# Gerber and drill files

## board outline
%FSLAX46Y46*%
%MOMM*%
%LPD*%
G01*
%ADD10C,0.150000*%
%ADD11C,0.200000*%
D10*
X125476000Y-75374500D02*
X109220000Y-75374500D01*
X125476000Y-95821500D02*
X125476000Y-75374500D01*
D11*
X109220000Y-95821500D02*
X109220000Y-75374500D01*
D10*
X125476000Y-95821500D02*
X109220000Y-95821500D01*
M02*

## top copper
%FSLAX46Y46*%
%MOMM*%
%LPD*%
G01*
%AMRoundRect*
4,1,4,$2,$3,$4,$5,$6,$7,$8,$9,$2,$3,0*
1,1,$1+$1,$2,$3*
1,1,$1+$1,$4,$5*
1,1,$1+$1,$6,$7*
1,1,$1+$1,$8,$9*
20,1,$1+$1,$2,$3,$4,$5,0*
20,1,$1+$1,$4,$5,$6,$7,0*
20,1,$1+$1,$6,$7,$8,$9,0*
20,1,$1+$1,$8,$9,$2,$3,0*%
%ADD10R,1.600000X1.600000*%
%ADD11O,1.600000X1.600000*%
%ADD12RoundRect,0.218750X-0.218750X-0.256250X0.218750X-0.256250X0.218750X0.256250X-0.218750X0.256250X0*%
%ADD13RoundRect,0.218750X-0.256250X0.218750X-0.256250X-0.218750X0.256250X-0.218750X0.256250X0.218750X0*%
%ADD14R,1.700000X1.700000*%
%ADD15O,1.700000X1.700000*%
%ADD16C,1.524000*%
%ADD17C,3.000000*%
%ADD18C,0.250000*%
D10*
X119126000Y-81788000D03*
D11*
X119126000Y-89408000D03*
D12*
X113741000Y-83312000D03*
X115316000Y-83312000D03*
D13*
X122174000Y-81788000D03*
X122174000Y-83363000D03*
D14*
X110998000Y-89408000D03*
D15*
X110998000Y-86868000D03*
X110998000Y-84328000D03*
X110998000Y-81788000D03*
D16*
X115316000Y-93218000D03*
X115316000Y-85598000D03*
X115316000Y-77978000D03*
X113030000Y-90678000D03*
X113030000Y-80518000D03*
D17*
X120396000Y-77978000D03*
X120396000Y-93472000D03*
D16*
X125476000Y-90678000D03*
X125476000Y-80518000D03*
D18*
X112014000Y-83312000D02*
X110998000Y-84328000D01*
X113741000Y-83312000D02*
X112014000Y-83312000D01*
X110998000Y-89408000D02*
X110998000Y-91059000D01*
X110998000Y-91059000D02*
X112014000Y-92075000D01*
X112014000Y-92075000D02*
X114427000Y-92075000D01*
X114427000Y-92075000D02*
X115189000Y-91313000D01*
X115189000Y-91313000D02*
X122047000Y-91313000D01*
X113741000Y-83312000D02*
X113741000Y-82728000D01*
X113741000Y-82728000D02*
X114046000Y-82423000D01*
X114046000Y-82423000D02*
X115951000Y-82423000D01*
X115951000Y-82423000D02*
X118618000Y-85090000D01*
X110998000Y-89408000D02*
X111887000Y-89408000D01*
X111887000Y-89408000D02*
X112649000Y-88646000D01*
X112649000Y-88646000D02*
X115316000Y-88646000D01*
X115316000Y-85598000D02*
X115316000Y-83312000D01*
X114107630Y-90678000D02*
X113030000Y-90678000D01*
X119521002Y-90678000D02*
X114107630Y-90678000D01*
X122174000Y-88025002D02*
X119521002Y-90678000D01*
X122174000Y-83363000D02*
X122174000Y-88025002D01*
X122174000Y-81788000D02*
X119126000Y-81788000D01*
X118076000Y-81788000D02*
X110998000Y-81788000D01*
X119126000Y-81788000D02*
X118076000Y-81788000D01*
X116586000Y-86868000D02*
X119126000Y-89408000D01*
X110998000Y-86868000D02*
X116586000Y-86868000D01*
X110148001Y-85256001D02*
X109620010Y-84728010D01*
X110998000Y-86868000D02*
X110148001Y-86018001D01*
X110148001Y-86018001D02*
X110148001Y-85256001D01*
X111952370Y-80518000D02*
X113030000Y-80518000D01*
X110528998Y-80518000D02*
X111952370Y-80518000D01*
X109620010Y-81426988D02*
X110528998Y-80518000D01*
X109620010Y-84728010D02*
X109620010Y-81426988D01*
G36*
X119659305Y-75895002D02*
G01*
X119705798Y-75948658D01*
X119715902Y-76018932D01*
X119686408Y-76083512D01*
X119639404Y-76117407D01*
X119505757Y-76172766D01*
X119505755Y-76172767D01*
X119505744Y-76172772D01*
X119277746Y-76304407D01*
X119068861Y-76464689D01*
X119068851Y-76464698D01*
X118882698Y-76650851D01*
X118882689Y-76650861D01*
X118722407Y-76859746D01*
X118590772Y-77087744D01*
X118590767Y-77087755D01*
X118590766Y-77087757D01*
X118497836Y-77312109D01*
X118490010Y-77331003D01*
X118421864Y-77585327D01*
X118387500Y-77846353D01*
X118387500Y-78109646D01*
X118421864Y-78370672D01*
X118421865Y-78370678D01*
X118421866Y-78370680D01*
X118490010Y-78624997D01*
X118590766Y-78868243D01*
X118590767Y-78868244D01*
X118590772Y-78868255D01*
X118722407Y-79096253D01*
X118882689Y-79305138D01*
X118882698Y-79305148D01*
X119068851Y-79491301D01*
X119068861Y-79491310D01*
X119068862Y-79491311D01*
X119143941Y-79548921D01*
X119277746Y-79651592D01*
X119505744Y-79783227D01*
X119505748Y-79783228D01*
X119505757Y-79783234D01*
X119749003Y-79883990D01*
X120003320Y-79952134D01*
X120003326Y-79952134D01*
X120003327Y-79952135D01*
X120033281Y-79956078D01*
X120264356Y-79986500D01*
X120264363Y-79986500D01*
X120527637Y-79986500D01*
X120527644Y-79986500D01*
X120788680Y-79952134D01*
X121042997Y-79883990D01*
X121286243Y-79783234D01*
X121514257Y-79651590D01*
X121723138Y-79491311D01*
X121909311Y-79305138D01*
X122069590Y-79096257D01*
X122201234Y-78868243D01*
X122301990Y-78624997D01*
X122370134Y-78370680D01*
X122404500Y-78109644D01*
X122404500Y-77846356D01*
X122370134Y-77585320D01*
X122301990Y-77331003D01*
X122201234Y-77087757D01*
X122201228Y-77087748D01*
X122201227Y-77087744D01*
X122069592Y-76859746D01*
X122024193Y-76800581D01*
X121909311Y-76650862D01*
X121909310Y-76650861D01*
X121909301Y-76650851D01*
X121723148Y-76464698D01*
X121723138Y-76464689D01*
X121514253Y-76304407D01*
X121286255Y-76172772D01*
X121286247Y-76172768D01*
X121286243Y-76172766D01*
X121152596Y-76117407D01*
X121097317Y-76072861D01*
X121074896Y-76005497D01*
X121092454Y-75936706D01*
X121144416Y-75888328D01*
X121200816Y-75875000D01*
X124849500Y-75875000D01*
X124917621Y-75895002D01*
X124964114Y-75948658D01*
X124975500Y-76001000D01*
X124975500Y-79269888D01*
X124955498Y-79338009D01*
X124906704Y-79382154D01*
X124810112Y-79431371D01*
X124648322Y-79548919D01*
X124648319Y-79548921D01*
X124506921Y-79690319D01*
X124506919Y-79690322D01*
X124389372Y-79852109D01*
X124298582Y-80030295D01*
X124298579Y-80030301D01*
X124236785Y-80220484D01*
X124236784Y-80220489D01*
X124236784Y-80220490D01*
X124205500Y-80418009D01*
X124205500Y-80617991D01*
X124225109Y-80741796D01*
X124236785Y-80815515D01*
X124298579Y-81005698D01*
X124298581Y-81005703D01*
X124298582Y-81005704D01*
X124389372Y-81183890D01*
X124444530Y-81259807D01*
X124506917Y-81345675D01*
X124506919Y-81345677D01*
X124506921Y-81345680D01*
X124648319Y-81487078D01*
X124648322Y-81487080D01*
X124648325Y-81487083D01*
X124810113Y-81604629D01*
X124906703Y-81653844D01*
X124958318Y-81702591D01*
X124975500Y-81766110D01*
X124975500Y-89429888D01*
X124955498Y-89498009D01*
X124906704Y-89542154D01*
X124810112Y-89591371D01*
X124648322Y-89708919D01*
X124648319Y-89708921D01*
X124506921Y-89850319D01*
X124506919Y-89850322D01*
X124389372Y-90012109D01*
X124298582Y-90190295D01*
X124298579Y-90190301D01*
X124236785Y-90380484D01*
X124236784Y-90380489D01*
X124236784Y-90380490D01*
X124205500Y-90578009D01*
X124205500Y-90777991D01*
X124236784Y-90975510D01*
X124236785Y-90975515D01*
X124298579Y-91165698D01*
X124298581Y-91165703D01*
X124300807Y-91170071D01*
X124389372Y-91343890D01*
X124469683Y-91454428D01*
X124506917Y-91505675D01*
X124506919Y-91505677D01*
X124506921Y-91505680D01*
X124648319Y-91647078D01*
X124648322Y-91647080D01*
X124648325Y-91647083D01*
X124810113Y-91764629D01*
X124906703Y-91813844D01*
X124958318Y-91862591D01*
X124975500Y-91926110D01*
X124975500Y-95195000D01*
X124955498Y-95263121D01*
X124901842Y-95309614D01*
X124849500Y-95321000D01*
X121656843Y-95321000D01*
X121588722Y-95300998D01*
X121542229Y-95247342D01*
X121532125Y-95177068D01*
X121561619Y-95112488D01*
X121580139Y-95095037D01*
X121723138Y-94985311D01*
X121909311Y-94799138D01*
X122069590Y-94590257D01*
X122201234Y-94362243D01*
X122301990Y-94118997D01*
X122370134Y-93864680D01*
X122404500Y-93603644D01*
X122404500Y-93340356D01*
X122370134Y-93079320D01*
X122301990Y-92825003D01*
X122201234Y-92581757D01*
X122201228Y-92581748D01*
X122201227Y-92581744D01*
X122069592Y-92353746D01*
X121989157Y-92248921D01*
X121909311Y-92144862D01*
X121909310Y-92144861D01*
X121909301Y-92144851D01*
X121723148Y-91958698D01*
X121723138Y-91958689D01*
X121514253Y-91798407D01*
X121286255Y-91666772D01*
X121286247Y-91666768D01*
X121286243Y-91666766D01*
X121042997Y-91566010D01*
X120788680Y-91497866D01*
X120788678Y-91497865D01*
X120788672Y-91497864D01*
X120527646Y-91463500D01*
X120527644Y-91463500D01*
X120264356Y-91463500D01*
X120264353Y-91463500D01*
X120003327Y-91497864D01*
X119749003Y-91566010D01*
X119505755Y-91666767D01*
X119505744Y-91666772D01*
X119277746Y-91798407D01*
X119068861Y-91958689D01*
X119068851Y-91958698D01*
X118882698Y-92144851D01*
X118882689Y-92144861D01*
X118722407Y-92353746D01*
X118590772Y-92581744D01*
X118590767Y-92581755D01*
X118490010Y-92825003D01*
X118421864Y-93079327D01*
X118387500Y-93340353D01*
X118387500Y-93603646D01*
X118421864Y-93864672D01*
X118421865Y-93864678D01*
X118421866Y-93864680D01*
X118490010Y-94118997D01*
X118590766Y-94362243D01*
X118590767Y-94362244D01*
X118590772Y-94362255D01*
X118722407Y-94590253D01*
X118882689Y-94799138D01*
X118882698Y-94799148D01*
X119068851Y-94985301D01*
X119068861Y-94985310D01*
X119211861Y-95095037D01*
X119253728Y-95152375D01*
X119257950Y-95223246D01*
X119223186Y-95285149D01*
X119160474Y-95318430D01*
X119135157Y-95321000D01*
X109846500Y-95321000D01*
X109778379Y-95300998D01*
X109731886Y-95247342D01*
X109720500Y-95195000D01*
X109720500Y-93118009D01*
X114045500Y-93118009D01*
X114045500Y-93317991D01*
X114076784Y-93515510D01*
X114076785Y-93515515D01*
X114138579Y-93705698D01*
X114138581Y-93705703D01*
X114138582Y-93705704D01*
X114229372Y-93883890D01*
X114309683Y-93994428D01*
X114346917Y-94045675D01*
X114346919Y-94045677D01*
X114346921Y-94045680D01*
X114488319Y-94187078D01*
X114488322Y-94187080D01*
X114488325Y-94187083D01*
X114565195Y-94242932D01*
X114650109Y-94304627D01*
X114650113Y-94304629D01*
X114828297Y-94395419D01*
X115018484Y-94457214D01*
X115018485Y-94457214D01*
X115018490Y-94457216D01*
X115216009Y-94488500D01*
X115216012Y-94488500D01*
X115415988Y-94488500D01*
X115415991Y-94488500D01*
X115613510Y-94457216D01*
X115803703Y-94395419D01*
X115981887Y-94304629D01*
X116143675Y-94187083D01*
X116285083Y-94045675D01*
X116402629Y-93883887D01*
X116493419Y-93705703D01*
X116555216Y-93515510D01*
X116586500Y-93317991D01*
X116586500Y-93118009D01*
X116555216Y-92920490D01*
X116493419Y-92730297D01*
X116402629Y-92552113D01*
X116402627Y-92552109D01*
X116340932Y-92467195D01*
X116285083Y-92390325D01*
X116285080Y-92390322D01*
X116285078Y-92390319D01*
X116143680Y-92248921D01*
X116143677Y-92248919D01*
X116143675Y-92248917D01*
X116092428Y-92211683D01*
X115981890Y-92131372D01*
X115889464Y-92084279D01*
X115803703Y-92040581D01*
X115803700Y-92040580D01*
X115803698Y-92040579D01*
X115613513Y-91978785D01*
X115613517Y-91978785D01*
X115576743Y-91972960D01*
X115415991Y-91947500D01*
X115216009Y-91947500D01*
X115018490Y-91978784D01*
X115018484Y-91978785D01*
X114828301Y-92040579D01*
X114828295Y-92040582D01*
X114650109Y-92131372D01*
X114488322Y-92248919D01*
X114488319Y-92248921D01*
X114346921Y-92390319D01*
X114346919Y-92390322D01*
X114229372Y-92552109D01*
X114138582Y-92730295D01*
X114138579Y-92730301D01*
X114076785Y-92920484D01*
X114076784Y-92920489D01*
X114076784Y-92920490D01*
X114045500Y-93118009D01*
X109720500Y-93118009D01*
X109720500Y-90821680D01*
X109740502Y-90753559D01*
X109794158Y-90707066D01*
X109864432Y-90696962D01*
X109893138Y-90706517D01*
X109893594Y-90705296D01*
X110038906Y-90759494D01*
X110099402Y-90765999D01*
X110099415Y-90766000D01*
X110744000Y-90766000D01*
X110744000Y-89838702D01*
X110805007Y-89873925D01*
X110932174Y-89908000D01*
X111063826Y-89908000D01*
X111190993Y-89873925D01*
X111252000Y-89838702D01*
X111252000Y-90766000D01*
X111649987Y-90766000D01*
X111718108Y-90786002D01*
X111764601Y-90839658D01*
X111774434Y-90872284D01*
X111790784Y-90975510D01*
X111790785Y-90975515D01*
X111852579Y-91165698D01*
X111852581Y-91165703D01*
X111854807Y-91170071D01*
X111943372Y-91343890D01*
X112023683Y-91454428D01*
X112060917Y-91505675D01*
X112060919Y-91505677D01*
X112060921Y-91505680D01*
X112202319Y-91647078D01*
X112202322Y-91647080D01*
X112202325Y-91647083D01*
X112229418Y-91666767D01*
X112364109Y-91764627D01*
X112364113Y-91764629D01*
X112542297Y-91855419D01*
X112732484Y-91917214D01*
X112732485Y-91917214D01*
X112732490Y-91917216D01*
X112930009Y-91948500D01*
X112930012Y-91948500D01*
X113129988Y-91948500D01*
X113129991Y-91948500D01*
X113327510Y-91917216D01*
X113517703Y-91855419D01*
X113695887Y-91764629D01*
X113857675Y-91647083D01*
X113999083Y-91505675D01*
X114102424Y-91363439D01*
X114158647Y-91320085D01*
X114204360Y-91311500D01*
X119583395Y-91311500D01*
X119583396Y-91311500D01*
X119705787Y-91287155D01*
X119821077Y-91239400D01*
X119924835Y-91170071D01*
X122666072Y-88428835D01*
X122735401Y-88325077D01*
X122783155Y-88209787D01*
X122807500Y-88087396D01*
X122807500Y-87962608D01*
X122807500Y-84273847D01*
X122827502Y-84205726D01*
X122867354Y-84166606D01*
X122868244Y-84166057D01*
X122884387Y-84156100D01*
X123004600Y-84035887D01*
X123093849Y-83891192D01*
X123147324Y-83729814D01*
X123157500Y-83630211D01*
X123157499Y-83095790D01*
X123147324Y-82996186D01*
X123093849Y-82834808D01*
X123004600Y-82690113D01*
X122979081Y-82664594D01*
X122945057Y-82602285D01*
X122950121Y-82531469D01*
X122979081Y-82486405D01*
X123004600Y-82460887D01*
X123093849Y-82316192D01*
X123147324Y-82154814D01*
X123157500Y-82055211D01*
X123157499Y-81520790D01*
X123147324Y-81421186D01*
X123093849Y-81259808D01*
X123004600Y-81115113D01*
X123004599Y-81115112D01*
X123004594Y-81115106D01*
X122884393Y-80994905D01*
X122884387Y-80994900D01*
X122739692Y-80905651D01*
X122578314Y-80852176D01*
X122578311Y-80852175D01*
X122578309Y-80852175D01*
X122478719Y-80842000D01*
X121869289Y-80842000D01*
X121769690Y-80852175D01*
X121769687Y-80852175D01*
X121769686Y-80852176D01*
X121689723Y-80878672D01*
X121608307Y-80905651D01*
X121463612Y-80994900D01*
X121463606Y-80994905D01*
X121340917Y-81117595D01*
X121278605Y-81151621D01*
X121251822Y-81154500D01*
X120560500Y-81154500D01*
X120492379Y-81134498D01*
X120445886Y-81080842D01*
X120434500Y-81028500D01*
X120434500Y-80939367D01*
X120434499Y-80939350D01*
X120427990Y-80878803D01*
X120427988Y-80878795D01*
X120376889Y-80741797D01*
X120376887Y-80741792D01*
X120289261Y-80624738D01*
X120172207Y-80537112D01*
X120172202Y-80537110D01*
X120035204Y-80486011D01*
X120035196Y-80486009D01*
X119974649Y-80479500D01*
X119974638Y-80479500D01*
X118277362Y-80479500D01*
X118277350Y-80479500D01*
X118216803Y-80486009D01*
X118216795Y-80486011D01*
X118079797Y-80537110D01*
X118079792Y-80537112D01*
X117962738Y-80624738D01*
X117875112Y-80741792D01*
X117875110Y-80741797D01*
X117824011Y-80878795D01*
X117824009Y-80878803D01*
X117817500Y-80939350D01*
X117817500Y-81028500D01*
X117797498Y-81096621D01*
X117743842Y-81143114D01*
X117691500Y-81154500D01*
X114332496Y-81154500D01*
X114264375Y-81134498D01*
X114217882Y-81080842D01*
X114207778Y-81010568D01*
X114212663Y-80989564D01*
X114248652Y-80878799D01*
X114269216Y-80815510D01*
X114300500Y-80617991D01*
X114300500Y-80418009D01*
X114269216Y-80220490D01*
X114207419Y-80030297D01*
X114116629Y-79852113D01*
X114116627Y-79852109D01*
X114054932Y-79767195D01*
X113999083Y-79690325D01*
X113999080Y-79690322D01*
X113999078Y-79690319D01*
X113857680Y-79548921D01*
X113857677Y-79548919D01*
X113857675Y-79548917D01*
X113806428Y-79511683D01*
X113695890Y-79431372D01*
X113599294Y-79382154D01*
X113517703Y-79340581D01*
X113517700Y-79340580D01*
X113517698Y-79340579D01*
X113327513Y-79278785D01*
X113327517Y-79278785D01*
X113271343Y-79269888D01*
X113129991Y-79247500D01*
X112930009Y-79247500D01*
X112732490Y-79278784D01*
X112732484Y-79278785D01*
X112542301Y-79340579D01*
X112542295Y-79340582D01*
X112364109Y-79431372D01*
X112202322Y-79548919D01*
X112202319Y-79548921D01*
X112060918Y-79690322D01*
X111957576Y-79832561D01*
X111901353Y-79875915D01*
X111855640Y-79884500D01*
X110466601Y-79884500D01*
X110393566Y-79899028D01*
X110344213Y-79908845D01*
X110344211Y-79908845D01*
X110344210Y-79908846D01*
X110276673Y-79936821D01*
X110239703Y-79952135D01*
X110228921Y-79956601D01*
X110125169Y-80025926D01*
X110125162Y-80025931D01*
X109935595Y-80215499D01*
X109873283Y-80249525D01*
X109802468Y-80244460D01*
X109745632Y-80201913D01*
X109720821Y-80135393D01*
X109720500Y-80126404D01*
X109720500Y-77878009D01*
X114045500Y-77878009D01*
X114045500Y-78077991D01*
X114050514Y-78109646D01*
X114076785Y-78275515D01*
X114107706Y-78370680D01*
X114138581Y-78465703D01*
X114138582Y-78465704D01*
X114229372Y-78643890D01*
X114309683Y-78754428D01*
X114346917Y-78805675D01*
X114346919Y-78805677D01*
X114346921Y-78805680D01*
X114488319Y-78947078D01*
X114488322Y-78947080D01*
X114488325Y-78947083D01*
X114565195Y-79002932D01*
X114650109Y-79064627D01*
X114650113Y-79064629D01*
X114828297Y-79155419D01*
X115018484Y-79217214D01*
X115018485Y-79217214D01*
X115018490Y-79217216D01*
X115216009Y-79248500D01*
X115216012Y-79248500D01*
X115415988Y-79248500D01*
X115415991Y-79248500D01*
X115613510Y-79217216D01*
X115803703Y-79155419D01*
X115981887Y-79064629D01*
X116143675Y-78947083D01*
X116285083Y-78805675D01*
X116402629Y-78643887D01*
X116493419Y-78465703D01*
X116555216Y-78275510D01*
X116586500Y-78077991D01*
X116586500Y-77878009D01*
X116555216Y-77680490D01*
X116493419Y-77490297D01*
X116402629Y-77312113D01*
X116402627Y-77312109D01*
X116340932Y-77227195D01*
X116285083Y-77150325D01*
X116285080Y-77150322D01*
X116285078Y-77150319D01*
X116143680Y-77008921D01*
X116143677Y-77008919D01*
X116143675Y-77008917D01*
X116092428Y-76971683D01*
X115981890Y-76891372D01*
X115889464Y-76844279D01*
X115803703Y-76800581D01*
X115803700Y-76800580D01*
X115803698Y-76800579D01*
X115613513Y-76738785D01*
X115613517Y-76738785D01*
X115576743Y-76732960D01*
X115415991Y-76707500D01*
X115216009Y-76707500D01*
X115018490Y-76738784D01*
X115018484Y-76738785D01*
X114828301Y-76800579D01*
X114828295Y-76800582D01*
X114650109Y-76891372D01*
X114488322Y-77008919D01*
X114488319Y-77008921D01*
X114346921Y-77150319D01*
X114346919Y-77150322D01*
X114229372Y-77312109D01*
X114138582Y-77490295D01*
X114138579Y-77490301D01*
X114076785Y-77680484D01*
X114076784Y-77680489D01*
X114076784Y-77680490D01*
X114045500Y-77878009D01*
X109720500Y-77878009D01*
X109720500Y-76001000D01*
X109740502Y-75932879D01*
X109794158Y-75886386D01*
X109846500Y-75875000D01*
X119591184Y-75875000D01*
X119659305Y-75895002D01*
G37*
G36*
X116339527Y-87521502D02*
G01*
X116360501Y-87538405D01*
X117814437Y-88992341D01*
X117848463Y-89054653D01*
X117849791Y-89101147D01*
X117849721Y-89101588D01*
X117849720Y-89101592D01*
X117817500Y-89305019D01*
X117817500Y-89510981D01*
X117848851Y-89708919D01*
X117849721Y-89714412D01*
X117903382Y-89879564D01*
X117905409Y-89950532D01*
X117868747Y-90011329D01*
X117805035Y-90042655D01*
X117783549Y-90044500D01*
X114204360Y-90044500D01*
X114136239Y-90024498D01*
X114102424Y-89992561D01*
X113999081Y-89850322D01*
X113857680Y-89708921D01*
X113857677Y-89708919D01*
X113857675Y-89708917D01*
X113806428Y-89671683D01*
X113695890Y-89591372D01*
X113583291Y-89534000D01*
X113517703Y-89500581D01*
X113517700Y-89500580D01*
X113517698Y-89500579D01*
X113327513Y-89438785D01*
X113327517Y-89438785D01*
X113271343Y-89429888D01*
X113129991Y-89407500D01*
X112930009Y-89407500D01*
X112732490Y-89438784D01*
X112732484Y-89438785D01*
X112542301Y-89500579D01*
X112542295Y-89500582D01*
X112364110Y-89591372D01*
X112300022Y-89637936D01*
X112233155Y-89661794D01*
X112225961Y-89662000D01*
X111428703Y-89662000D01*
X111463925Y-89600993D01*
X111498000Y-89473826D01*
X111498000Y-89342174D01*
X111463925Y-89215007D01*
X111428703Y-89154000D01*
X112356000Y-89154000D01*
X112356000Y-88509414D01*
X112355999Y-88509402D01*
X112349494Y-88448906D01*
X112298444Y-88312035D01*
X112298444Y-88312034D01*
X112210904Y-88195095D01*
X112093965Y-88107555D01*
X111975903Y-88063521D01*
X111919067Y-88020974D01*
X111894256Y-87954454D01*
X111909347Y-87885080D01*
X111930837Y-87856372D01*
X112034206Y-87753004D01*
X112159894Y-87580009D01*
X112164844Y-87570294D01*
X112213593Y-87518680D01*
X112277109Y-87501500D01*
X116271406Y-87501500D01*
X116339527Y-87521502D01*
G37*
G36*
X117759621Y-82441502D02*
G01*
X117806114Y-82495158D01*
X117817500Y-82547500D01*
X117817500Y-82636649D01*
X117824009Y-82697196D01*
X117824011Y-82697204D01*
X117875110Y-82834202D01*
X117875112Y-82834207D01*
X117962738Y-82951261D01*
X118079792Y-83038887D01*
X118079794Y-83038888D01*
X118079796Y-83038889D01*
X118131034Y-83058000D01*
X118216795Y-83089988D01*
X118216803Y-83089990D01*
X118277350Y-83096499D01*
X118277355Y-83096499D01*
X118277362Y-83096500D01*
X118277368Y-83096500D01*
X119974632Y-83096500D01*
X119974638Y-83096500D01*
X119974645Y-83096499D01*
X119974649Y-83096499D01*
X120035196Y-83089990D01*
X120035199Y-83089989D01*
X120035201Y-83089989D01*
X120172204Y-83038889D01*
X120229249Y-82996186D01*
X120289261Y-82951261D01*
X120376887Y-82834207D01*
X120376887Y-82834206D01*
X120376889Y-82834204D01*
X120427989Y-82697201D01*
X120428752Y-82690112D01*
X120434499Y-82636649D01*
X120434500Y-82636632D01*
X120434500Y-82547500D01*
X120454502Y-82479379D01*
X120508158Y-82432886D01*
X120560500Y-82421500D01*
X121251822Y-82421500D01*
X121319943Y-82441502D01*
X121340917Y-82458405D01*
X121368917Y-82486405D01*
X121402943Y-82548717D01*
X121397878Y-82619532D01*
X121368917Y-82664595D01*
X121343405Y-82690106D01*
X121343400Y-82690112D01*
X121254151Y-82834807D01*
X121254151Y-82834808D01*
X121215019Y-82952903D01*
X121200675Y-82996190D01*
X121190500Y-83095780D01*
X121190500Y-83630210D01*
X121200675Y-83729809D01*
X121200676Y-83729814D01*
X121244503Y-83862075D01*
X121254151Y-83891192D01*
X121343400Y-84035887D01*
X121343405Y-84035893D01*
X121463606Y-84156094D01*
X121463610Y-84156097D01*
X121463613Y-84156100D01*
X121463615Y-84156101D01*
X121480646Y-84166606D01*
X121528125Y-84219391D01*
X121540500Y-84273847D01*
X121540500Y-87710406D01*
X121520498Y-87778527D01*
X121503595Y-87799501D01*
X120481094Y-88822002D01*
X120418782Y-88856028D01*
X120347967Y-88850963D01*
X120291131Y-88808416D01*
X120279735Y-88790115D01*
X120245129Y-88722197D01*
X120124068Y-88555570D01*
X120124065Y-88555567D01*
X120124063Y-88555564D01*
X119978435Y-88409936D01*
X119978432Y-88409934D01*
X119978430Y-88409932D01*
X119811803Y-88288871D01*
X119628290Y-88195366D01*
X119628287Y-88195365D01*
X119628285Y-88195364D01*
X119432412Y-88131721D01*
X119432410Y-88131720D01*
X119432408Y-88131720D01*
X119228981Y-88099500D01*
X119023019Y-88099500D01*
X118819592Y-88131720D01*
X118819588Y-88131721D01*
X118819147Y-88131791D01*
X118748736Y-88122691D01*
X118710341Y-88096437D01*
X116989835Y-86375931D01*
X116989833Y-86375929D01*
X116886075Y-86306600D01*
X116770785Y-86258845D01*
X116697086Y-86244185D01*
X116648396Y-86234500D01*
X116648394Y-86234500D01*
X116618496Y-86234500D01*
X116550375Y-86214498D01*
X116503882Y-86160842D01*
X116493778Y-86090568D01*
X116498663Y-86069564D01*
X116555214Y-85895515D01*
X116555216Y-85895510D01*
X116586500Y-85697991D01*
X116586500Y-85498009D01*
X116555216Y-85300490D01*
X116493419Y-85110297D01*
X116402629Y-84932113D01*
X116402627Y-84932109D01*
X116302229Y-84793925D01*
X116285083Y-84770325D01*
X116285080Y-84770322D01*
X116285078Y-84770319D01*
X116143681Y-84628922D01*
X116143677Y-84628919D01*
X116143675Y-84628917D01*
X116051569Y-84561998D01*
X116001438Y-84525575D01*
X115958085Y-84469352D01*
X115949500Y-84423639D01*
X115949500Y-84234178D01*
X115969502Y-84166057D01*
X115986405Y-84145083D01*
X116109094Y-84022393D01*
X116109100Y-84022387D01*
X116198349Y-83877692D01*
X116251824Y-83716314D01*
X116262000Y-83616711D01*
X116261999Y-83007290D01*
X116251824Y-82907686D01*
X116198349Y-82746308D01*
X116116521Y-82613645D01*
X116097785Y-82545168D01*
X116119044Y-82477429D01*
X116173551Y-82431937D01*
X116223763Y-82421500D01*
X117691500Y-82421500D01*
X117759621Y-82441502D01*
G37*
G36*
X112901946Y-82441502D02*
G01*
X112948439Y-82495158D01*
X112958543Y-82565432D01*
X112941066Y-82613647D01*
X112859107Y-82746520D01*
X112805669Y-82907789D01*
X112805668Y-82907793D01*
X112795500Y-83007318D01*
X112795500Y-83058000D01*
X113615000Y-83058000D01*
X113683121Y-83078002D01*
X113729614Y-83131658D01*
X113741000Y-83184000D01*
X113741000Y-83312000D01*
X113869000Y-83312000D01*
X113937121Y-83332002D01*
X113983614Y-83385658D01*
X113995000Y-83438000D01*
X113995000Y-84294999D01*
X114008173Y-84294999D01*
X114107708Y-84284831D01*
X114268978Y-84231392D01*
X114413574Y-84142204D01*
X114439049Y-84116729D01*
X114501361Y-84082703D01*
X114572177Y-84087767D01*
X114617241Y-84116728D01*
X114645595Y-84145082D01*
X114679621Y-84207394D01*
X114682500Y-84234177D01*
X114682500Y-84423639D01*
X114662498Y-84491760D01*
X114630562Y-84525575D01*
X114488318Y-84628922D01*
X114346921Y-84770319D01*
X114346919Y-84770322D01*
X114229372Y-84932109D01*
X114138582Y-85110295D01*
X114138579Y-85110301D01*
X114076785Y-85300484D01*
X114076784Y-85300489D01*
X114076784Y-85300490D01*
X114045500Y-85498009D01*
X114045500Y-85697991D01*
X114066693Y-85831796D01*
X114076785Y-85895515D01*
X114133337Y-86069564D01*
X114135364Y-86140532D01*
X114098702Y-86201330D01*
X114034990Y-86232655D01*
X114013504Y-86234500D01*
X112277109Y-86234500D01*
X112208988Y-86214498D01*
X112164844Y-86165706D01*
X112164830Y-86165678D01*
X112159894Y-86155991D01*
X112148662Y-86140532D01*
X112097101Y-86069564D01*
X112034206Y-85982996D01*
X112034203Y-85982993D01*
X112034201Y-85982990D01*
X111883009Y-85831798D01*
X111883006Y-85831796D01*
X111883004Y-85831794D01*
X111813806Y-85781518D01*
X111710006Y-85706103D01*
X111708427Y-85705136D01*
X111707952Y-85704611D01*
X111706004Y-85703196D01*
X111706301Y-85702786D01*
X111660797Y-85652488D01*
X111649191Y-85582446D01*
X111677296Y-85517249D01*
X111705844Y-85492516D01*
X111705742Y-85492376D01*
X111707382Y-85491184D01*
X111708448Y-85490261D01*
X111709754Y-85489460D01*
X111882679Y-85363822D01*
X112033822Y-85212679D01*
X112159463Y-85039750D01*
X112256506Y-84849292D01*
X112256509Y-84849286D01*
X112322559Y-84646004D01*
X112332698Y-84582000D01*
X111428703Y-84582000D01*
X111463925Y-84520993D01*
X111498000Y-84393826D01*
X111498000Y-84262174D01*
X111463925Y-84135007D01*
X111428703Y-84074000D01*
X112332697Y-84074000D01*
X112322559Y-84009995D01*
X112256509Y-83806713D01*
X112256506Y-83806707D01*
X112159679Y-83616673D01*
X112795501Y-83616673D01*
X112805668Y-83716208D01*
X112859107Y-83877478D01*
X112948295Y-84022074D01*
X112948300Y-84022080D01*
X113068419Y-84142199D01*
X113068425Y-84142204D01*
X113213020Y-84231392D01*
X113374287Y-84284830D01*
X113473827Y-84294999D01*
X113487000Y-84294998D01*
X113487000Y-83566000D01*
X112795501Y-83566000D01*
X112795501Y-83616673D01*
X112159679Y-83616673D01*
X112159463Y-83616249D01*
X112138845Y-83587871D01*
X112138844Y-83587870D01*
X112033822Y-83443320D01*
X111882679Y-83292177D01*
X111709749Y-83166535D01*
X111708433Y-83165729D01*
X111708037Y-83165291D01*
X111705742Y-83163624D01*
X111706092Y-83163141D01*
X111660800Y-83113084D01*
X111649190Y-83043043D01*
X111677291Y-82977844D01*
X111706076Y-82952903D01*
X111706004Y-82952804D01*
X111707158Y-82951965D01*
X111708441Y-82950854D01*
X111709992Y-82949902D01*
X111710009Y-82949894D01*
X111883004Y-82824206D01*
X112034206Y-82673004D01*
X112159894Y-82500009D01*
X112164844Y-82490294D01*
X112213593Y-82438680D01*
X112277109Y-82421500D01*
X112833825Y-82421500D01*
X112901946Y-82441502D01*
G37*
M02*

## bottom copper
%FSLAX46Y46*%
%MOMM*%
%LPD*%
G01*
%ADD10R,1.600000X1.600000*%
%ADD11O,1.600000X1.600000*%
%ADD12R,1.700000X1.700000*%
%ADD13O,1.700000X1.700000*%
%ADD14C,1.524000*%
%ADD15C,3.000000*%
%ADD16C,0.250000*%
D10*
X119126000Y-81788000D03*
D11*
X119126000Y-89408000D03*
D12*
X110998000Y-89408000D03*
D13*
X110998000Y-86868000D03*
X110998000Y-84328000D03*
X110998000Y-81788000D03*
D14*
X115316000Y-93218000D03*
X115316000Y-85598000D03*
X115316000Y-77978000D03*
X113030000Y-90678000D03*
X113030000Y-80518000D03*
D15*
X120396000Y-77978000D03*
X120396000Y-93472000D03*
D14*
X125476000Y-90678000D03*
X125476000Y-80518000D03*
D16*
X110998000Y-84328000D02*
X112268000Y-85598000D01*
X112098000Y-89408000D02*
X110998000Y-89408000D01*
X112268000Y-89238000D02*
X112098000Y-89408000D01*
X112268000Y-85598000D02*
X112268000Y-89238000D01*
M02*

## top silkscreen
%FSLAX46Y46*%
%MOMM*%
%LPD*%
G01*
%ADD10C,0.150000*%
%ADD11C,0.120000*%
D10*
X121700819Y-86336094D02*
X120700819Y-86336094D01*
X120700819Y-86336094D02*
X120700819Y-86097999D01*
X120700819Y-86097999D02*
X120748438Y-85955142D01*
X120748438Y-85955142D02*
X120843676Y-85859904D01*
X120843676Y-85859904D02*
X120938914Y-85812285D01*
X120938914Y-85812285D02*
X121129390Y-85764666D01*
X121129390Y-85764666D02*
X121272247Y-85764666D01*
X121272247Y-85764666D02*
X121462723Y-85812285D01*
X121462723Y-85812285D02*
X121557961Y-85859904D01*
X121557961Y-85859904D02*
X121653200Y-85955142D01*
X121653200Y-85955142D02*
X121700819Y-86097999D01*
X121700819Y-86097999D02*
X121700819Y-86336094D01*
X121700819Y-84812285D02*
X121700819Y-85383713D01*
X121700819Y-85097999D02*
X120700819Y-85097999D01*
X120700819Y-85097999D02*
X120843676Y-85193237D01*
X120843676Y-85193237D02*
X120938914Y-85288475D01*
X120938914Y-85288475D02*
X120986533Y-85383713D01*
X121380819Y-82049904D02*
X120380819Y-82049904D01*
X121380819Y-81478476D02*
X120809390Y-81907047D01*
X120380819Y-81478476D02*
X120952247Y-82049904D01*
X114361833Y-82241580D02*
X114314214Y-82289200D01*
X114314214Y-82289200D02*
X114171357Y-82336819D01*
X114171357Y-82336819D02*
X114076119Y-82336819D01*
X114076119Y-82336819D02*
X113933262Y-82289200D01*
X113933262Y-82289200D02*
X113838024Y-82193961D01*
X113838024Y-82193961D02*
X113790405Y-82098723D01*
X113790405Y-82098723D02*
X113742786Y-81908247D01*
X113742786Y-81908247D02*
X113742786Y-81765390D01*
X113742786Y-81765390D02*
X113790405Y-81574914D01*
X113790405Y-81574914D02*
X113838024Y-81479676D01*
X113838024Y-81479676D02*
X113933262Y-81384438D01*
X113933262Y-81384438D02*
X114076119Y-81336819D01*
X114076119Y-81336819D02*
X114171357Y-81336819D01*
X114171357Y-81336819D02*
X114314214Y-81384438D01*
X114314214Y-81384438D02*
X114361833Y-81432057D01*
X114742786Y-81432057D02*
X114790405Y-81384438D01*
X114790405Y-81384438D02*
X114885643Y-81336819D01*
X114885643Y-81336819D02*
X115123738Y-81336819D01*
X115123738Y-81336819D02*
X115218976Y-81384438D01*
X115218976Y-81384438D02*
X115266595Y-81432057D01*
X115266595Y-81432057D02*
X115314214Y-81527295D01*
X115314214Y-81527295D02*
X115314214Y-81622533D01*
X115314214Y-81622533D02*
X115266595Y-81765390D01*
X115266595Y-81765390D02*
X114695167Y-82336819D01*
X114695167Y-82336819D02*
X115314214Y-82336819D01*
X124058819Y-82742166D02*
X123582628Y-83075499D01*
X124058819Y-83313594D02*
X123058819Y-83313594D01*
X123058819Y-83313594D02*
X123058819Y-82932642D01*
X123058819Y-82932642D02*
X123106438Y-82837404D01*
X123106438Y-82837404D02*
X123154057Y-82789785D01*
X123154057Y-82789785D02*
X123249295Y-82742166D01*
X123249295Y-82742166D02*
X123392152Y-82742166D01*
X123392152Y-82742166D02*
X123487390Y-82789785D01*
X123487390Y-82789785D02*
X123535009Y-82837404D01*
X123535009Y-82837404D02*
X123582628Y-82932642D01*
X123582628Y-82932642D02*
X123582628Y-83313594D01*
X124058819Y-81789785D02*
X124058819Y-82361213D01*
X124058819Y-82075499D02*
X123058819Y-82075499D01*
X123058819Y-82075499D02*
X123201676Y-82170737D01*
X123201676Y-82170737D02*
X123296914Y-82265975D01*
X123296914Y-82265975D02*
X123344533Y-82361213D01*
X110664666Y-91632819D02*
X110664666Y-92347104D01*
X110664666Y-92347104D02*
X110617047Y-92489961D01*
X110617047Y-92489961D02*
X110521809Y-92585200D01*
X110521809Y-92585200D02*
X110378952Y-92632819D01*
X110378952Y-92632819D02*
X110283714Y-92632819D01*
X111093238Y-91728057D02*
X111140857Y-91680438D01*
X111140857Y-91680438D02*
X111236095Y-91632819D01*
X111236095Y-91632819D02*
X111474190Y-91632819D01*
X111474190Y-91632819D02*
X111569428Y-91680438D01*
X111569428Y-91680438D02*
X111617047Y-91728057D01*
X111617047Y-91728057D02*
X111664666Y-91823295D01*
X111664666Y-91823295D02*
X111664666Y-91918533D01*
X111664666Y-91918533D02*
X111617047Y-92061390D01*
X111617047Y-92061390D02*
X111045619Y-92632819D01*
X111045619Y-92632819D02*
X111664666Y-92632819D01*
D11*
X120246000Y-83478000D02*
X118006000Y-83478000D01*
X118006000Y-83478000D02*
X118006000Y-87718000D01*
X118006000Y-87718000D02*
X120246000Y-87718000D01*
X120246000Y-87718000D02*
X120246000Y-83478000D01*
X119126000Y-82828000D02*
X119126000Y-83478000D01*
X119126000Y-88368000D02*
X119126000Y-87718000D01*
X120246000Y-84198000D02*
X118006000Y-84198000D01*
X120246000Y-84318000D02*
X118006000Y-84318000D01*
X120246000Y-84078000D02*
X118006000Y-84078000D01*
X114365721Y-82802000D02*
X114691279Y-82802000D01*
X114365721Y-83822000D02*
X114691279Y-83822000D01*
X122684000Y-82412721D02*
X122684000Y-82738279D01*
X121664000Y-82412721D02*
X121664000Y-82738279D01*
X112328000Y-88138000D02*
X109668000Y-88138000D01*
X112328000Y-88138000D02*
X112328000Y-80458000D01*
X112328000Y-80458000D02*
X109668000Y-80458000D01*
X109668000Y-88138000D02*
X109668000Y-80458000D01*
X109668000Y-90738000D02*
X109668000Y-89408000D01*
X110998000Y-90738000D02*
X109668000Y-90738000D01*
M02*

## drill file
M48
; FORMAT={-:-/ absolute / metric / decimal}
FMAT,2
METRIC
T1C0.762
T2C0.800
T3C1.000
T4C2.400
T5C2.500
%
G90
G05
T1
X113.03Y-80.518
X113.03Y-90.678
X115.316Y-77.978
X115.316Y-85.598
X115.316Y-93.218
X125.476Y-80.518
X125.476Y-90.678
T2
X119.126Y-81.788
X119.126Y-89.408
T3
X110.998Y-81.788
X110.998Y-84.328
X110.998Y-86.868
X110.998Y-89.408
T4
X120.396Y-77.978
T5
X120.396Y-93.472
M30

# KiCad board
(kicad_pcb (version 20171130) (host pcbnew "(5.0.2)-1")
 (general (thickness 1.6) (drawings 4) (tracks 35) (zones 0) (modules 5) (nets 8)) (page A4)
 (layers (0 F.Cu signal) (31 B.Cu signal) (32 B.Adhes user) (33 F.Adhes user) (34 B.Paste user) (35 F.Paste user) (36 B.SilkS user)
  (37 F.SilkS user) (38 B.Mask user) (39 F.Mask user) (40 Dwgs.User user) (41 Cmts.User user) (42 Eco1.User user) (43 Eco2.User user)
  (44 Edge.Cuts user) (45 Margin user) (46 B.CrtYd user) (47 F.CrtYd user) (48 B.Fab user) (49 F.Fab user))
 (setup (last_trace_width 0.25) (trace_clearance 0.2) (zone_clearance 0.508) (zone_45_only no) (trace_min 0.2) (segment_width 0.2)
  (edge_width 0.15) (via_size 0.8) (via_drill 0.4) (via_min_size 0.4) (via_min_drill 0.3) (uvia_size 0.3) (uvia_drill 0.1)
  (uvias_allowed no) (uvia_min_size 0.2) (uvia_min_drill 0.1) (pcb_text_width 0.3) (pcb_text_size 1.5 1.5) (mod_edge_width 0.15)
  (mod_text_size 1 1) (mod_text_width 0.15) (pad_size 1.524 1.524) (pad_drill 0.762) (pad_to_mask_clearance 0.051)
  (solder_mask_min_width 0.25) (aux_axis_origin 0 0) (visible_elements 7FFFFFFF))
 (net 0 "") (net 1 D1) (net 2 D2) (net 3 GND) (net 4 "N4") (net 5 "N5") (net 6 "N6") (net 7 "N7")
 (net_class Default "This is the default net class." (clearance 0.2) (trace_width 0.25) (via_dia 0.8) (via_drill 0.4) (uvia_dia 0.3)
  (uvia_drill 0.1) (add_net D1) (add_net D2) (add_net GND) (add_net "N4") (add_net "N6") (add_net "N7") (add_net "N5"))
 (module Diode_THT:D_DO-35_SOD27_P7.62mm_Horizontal (layer F.Cu) (at 119.126 81.788 270)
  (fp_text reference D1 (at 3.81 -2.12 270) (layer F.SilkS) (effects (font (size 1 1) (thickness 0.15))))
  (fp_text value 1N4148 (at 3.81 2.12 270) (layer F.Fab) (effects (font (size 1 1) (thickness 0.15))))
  (fp_line (start 1.69 -1.12) (end 1.69 1.12) (layer F.SilkS) (width 0.12))
  (fp_line (start 1.69 1.12) (end 5.93 1.12) (layer F.SilkS) (width 0.12))
  (fp_line (start 5.93 1.12) (end 5.93 -1.12) (layer F.SilkS) (width 0.12))
  (fp_line (start 5.93 -1.12) (end 1.69 -1.12) (layer F.SilkS) (width 0.12))
  (fp_line (start 1.04 0) (end 1.69 0) (layer F.SilkS) (width 0.12))
  (fp_line (start 6.58 0) (end 5.93 0) (layer F.SilkS) (width 0.12))
  (fp_line (start 2.41 -1.12) (end 2.41 1.12) (layer F.SilkS) (width 0.12))
  (fp_line (start 2.53 -1.12) (end 2.53 1.12) (layer F.SilkS) (width 0.12))
  (fp_line (start 2.29 -1.12) (end 2.29 1.12) (layer F.SilkS) (width 0.12))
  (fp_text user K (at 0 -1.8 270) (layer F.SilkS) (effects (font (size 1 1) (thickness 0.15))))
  (pad 1 thru_hole rect (at 0 0 270) (size 1.6 1.6) (drill 0.8) (layers *.Cu *.Mask) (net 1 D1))
  (pad 2 thru_hole oval (at 7.62 0 270) (size 1.6 1.6) (drill 0.8) (layers *.Cu *.Mask) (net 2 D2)))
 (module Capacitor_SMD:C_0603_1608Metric (layer F.Cu) (at 114.5285 83.312)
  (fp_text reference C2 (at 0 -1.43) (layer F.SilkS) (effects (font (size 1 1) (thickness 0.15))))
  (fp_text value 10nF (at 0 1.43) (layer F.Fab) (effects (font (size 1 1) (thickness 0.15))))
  (fp_line (start -0.162779 -0.51) (end 0.162779 -0.51) (layer F.SilkS) (width 0.12))
  (fp_line (start -0.162779 0.51) (end 0.162779 0.51) (layer F.SilkS) (width 0.12))
  (pad 1 smd roundrect (at -0.7875 0) (size 0.875 0.95) (layers F.Cu F.Paste F.Mask) (roundrect_rratio 0.25) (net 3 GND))
  (pad 2 smd roundrect (at 0.7875 0) (size 0.875 0.95) (layers F.Cu F.Paste F.Mask) (roundrect_rratio 0.25) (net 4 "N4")))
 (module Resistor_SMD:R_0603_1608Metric (layer F.Cu) (at 122.174 82.5755 270)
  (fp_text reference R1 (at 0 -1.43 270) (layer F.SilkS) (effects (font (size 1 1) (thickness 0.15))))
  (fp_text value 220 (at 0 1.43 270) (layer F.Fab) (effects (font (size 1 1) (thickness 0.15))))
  (fp_line (start -0.162779 -0.51) (end 0.162779 -0.51) (layer F.SilkS) (width 0.12))
  (fp_line (start -0.162779 0.51) (end 0.162779 0.51) (layer F.SilkS) (width 0.12))
  (pad 1 smd roundrect (at -0.7875 0 270) (size 0.875 0.95) (layers F.Cu F.Paste F.Mask) (roundrect_rratio 0.25) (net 1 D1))
  (pad 2 smd roundrect (at 0.7875 0 270) (size 0.875 0.95) (layers F.Cu F.Paste F.Mask) (roundrect_rratio 0.25) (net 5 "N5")))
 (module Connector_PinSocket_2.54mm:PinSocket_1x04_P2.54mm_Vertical (layer F.Cu) (at 110.998 89.408 180)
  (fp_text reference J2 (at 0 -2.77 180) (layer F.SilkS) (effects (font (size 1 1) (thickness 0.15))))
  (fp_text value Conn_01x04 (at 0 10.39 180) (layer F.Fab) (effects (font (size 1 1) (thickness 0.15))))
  (fp_line (start -1.33 1.27) (end 1.33 1.27) (layer F.SilkS) (width 0.12))
  (fp_line (start -1.33 1.27) (end -1.33 8.95) (layer F.SilkS) (width 0.12))
  (fp_line (start -1.33 8.95) (end 1.33 8.95) (layer F.SilkS) (width 0.12))
  (fp_line (start 1.33 1.27) (end 1.33 8.95) (layer F.SilkS) (width 0.12))
  (fp_line (start 1.33 -1.33) (end 1.33 0) (layer F.SilkS) (width 0.12))
  (fp_line (start 0 -1.33) (end 1.33 -1.33) (layer F.SilkS) (width 0.12))
  (pad 1 thru_hole rect (at 0 0 180) (size 1.7 1.7) (drill 1) (layers *.Cu *.Mask) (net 3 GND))
  (pad 2 thru_hole oval (at 0 2.54 180) (size 1.7 1.7) (drill 1) (layers *.Cu *.Mask) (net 2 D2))
  (pad 3 thru_hole oval (at 0 5.08 180) (size 1.7 1.7) (drill 1) (layers *.Cu *.Mask) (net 3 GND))
  (pad 4 thru_hole oval (at 0 7.62 180) (size 1.7 1.7) (drill 1) (layers *.Cu *.Mask) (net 1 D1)))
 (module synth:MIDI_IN (layer B.Cu) (at 115.316 85.598 270)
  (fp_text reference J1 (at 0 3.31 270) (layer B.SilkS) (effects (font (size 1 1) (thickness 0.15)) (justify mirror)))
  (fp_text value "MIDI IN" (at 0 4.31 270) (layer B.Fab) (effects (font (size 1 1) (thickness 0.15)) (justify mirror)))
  (pad 1 thru_hole circle (at 7.62 0 270) (size 1.524 1.524) (drill 0.762) (layers *.Cu *.Mask) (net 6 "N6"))
  (pad 2 thru_hole circle (at 0 0 270) (size 1.524 1.524) (drill 0.762) (layers *.Cu *.Mask) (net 4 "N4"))
  (pad 3 thru_hole circle (at -7.62 0 270) (size 1.524 1.524) (drill 0.762) (layers *.Cu *.Mask) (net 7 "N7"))
  (pad 4 thru_hole circle (at 5.08 2.286 270) (size 1.524 1.524) (drill 0.762) (layers *.Cu *.Mask) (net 5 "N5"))
  (pad 5 thru_hole circle (at -5.08 2.286 270) (size 1.524 1.524) (drill 0.762) (layers *.Cu *.Mask) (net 2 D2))
  (pad "" thru_hole circle (at -7.62 -5.08 270) (size 3 3) (drill 2.4) (layers *.Cu *.Mask))
  (pad "" thru_hole circle (at 7.874 -5.08 270) (size 3 3) (drill 2.5) (layers *.Cu *.Mask))
  (pad "" thru_hole circle (at 5.08 -10.16 270) (size 1.524 1.524) (drill 0.762) (layers *.Cu *.Mask))
  (pad "" thru_hole circle (at -5.08 -10.16 270) (size 1.524 1.524) (drill 0.762) (layers *.Cu *.Mask)))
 (gr_line (start 125.476 75.3745) (end 109.22 75.3745) (layer Edge.Cuts) (width 0.15))
 (gr_line (start 125.476 95.8215) (end 125.476 75.3745) (layer Edge.Cuts) (width 0.15))
 (gr_line (start 109.22 95.8215) (end 109.22 75.3745) (layer Edge.Cuts) (width 0.2))
 (gr_line (start 125.476 95.8215) (end 109.22 95.8215) (layer Edge.Cuts) (width 0.15))
 (segment (start 112.014 83.312) (end 110.998 84.328) (width 0.25) (layer F.Cu) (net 3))
 (segment (start 113.741 83.312) (end 112.014 83.312) (width 0.25) (layer F.Cu) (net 3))
 (segment (start 110.998 84.328) (end 112.268 85.598) (width 0.25) (layer B.Cu) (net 3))
 (segment (start 112.098 89.408) (end 110.998 89.408) (width 0.25) (layer B.Cu) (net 3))
 (segment (start 112.268 89.238) (end 112.098 89.408) (width 0.25) (layer B.Cu) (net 3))
 (segment (start 112.268 85.598) (end 112.268 89.238) (width 0.25) (layer B.Cu) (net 3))
 (segment (start 110.998 89.408) (end 110.998 91.059) (width 0.25) (layer F.Cu) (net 3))
 (segment (start 110.998 91.059) (end 112.014 92.075) (width 0.25) (layer F.Cu) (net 3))
 (segment (start 112.014 92.075) (end 114.427 92.075) (width 0.25) (layer F.Cu) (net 3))
 (segment (start 114.427 92.075) (end 115.189 91.313) (width 0.25) (layer F.Cu) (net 3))
 (segment (start 115.189 91.313) (end 122.047 91.313) (width 0.25) (layer F.Cu) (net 3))
 (segment (start 113.741 83.312) (end 113.741 82.728) (width 0.25) (layer F.Cu) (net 3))
 (segment (start 113.741 82.728) (end 114.046 82.423) (width 0.25) (layer F.Cu) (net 3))
 (segment (start 114.046 82.423) (end 115.951 82.423) (width 0.25) (layer F.Cu) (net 3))
 (segment (start 115.951 82.423) (end 118.618 85.09) (width 0.25) (layer F.Cu) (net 3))
 (segment (start 110.998 89.408) (end 111.887 89.408) (width 0.25) (layer F.Cu) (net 3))
 (segment (start 111.887 89.408) (end 112.649 88.646) (width 0.25) (layer F.Cu) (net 3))
 (segment (start 112.649 88.646) (end 115.316 88.646) (width 0.25) (layer F.Cu) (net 3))
 (segment (start 115.316 85.598) (end 115.316 83.312) (width 0.25) (layer F.Cu) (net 4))
 (segment (start 114.10763 90.678) (end 113.03 90.678) (width 0.25) (layer F.Cu) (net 5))
 (segment (start 119.521002 90.678) (end 114.10763 90.678) (width 0.25) (layer F.Cu) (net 5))
 (segment (start 122.174 88.025002) (end 119.521002 90.678) (width 0.25) (layer F.Cu) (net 5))
 (segment (start 122.174 83.363) (end 122.174 88.025002) (width 0.25) (layer F.Cu) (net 5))
 (segment (start 122.174 81.788) (end 119.126 81.788) (width 0.25) (layer F.Cu) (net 1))
 (segment (start 118.076 81.788) (end 110.998 81.788) (width 0.25) (layer F.Cu) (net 1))
 (segment (start 119.126 81.788) (end 118.076 81.788) (width 0.25) (layer F.Cu) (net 1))
 (segment (start 116.586 86.868) (end 119.126 89.408) (width 0.25) (layer F.Cu) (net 2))
 (segment (start 110.998 86.868) (end 116.586 86.868) (width 0.25) (layer F.Cu) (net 2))
 (segment (start 110.148001 85.256001) (end 109.62001 84.72801) (width 0.25) (layer F.Cu) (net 2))
 (segment (start 110.998 86.868) (end 110.148001 86.018001) (width 0.25) (layer F.Cu) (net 2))
 (segment (start 110.148001 86.018001) (end 110.148001 85.256001) (width 0.25) (layer F.Cu) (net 2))
 (segment (start 111.95237 80.518) (end 113.03 80.518) (width 0.25) (layer F.Cu) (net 2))
 (segment (start 110.528998 80.518) (end 111.95237 80.518) (width 0.25) (layer F.Cu) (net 2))
 (segment (start 109.62001 81.426988) (end 110.528998 80.518) (width 0.25) (layer F.Cu) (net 2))
 (segment (start 109.62001 84.72801) (end 109.62001 81.426988) (width 0.25) (layer F.Cu) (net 2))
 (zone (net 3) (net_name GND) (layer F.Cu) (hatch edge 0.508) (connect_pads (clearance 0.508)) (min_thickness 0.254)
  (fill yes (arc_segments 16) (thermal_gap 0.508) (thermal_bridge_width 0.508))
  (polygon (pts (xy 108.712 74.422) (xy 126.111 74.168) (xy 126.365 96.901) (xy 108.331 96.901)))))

